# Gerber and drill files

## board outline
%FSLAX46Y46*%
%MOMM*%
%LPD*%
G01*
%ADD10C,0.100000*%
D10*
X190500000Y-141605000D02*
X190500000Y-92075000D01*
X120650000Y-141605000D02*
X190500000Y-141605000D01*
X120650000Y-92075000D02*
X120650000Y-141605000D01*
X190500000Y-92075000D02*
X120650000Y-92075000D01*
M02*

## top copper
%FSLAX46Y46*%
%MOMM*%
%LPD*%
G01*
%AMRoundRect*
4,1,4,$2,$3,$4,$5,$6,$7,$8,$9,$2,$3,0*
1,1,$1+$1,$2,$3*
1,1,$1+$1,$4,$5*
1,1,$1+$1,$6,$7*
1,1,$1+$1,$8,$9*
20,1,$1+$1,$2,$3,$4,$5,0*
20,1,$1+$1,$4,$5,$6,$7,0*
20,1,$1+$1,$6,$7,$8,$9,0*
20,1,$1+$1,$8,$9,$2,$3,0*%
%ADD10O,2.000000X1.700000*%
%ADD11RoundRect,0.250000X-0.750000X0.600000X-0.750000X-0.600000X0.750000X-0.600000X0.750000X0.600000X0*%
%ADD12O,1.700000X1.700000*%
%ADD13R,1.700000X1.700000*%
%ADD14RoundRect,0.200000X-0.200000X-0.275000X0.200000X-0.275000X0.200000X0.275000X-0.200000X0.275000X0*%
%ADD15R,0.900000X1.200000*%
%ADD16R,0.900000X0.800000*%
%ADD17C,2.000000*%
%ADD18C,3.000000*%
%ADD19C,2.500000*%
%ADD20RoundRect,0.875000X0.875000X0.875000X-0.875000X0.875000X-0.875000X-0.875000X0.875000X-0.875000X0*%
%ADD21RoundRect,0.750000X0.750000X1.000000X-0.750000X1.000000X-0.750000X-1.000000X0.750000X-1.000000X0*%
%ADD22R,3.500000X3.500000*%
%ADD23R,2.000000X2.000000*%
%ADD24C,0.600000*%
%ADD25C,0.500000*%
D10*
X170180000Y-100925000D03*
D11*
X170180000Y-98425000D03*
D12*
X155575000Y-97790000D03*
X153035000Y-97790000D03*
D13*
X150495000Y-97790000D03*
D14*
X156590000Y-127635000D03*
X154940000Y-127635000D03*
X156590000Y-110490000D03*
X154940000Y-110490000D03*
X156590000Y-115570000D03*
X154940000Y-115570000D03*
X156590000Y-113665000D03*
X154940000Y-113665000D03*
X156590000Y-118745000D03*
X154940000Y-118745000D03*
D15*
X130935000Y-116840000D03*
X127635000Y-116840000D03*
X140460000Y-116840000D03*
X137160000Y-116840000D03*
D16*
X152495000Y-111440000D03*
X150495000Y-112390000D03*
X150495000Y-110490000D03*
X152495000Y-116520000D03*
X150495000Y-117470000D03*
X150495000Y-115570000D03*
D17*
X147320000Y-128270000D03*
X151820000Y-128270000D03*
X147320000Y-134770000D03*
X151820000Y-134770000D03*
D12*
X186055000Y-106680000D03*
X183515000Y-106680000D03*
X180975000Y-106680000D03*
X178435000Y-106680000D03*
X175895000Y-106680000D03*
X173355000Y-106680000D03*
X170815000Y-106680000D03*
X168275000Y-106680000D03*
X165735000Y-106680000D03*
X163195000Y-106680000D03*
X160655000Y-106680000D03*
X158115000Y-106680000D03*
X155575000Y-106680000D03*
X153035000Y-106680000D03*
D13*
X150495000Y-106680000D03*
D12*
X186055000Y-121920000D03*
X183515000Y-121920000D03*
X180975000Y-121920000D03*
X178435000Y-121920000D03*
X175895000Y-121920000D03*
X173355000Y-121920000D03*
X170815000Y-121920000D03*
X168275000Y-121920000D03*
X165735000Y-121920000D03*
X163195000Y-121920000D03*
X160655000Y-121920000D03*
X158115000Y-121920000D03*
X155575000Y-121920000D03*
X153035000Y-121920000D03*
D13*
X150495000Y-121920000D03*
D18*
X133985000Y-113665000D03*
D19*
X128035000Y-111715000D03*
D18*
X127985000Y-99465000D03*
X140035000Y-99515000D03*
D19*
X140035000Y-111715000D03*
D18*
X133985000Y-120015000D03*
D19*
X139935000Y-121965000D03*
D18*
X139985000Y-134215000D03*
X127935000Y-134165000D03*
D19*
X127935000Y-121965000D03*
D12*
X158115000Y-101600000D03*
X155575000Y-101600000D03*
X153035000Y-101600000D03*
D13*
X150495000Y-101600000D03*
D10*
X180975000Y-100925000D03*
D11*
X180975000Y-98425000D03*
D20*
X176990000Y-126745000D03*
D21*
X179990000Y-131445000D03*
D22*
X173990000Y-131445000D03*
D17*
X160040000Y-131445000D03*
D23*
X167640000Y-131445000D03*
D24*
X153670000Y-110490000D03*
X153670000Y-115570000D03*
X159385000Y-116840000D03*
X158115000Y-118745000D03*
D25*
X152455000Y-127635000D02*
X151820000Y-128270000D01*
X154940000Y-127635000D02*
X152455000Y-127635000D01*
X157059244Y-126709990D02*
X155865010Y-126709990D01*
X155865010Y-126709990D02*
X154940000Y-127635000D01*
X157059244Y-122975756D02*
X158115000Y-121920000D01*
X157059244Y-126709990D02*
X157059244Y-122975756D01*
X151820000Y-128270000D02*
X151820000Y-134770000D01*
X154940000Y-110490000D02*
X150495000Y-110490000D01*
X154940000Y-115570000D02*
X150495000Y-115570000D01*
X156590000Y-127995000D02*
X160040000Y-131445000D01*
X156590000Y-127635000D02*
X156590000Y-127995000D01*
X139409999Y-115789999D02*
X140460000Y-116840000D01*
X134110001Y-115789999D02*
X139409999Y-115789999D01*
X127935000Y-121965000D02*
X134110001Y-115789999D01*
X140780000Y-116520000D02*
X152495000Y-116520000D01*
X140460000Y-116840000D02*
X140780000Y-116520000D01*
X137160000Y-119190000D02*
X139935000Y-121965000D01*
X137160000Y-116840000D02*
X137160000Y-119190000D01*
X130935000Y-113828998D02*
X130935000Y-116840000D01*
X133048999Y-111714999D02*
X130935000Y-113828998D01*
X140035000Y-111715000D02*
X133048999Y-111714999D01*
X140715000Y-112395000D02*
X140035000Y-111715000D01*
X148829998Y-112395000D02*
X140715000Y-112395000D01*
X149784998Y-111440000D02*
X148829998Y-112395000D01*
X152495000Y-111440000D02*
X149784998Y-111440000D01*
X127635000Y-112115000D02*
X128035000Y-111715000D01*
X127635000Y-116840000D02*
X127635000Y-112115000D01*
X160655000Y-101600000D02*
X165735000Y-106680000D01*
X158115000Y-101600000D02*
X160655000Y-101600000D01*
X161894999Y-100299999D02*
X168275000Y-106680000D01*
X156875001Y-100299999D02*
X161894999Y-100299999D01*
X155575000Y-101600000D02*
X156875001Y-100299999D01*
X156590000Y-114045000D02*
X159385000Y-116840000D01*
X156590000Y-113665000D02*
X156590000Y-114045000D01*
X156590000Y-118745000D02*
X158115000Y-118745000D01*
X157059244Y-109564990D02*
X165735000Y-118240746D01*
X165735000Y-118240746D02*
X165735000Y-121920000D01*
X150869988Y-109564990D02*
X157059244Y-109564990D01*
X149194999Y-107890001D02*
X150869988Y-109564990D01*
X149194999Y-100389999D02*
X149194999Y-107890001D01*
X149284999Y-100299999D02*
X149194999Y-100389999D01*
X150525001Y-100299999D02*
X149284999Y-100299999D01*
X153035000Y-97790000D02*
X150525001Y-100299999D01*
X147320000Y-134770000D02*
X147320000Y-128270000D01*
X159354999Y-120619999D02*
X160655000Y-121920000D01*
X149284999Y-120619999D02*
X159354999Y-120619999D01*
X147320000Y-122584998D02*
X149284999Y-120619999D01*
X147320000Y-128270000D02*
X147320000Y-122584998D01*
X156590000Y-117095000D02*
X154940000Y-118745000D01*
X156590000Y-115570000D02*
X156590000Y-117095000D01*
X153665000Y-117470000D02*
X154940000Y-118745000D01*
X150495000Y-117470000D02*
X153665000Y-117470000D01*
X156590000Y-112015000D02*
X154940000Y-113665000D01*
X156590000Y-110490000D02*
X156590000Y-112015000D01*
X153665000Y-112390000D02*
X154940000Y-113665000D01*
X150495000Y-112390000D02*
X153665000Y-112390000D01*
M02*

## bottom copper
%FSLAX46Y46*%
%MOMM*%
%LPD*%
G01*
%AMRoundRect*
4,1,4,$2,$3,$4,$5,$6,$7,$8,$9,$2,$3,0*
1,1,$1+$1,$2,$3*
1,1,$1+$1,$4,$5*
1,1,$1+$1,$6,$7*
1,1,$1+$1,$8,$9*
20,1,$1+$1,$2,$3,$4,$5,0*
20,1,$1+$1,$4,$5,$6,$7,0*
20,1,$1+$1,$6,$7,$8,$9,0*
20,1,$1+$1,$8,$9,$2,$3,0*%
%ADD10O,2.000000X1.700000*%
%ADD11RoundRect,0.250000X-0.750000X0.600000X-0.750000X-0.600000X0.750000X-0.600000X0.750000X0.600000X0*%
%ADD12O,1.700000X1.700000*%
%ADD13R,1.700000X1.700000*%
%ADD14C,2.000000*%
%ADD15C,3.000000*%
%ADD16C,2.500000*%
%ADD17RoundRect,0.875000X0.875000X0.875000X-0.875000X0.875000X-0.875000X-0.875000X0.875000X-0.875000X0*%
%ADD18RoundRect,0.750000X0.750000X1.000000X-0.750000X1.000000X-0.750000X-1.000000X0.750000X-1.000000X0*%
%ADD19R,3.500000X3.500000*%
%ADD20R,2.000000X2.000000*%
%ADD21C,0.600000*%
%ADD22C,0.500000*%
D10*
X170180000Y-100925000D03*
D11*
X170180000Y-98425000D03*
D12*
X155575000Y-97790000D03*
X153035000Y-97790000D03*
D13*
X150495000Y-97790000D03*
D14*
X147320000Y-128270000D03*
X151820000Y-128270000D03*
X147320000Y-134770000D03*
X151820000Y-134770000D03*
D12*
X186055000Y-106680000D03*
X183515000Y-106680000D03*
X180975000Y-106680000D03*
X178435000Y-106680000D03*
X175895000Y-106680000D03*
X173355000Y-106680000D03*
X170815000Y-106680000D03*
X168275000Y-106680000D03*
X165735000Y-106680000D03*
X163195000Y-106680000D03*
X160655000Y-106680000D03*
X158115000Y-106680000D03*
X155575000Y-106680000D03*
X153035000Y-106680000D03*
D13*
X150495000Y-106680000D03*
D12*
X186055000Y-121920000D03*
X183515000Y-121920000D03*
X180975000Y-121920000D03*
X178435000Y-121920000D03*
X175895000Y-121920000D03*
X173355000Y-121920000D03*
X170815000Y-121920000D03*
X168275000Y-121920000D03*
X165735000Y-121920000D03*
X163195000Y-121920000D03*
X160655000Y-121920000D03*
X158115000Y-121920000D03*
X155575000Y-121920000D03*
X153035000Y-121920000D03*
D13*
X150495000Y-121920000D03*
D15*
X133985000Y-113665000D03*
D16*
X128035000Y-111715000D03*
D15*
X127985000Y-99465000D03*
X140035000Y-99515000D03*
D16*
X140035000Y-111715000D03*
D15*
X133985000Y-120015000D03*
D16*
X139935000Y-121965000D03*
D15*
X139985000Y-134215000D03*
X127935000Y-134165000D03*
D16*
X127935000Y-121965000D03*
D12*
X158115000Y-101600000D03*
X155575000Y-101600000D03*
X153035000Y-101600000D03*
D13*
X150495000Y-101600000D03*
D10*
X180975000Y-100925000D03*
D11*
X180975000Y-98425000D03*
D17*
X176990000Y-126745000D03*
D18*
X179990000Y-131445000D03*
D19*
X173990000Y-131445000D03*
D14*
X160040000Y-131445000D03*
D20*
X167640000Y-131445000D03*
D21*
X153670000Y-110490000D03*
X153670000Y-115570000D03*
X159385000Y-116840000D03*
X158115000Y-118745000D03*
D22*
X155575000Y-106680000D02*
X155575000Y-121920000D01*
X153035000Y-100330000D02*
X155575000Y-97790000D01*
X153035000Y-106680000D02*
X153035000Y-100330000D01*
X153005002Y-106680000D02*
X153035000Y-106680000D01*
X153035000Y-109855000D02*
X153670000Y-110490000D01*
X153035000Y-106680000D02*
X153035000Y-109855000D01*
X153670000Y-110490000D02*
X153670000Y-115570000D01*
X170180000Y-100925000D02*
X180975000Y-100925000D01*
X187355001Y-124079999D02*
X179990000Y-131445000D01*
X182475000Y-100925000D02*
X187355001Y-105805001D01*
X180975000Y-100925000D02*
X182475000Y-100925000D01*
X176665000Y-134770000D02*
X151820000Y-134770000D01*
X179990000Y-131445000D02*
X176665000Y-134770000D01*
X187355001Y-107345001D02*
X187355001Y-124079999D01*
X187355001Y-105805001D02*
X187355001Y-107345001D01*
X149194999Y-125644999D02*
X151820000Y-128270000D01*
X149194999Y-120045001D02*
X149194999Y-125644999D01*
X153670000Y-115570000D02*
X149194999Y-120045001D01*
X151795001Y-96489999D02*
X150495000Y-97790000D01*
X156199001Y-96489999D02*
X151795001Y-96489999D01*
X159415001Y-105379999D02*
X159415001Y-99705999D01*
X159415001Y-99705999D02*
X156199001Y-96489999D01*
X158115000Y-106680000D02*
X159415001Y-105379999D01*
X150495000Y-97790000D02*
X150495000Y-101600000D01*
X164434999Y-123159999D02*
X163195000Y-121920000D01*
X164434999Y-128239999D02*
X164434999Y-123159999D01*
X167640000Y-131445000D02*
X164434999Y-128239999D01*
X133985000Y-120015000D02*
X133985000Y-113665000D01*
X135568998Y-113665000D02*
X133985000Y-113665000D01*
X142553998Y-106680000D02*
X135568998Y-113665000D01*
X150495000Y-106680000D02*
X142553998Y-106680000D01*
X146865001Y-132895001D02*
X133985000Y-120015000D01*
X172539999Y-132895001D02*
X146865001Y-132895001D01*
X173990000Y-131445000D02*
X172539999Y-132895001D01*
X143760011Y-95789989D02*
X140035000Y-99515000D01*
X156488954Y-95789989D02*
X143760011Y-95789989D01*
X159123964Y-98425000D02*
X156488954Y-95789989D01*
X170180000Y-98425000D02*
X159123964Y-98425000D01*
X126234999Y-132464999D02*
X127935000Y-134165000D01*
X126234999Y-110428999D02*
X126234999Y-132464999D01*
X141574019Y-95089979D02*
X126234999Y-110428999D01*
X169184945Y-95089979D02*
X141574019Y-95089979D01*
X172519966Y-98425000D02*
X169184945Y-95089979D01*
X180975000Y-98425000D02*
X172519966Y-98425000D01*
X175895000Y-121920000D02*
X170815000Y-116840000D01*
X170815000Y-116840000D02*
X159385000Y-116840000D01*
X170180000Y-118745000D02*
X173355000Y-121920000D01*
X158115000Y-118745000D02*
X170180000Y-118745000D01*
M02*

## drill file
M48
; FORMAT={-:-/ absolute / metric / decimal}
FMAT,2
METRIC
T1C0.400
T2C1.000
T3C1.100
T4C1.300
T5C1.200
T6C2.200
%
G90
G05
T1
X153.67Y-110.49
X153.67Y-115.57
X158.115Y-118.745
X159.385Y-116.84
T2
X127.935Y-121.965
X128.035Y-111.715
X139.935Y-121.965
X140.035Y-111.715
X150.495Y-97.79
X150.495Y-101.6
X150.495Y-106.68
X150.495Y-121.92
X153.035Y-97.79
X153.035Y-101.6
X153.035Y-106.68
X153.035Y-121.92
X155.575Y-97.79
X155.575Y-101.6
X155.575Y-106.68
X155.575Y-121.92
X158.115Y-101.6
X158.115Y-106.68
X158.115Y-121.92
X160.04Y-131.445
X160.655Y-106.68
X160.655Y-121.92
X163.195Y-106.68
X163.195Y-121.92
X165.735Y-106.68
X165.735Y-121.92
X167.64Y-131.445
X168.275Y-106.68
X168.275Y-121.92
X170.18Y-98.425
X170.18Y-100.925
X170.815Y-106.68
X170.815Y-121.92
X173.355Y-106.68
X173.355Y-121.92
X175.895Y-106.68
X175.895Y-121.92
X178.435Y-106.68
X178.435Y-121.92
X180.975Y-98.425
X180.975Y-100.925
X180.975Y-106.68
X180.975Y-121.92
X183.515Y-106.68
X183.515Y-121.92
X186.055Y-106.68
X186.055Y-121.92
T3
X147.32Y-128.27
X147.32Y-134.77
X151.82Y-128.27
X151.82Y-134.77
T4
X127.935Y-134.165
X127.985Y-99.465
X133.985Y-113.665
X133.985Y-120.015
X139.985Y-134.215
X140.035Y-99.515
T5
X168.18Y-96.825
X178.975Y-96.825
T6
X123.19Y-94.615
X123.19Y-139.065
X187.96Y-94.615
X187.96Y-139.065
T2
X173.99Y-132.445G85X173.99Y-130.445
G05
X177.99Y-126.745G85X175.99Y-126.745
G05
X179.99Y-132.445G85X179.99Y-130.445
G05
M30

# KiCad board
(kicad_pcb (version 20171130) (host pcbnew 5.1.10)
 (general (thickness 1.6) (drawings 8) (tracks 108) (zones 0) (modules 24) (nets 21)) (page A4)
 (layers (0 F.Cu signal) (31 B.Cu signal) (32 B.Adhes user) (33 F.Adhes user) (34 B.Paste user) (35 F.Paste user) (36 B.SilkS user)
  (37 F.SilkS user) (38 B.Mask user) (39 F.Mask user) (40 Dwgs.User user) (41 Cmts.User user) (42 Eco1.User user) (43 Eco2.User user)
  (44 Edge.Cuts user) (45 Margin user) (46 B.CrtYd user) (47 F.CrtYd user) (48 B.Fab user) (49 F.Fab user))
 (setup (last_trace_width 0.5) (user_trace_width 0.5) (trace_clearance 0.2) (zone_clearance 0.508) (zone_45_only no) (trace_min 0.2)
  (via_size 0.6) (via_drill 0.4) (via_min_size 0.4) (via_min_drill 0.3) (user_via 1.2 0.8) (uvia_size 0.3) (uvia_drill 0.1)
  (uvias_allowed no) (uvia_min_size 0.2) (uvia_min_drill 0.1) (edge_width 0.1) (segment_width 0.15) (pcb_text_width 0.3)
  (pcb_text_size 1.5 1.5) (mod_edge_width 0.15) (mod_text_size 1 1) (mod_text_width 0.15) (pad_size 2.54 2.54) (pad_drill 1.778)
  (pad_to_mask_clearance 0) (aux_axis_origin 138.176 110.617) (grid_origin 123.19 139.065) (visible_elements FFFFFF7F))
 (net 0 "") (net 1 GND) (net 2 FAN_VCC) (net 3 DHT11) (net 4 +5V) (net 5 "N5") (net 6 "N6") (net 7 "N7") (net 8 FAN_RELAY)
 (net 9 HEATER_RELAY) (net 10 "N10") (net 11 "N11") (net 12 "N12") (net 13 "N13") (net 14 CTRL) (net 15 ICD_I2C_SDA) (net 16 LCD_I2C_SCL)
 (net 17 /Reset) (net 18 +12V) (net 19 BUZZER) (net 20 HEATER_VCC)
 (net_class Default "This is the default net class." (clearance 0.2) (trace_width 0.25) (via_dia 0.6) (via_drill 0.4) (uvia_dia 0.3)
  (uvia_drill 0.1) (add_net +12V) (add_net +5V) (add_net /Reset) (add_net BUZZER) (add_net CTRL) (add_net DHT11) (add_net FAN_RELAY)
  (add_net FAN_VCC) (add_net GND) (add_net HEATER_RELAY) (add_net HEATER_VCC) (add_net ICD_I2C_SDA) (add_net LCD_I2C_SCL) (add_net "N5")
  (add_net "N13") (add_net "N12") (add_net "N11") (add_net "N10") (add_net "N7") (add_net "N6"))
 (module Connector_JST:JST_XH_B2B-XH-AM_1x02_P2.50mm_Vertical (layer F.Cu) (at 170.18 98.425 270)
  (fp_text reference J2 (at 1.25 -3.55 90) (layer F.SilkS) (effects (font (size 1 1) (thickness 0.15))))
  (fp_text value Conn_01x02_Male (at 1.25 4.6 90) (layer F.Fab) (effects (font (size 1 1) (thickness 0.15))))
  (pad "" np_thru_hole circle (at -1.6 2 270) (size 1.2 1.2) (drill 1.2) (layers *.Cu *.Mask))
  (pad 2 thru_hole oval (at 2.5 0 270) (size 1.7 2) (drill 1) (layers *.Cu *.Mask) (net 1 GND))
  (pad 1 thru_hole roundrect (at 0 0 270) (size 1.7 2) (drill 1) (layers *.Cu *.Mask) (roundrect_rratio 0.147059) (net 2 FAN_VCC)))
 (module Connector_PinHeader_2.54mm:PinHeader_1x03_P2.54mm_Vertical (layer F.Cu) (at 150.495 97.79 90)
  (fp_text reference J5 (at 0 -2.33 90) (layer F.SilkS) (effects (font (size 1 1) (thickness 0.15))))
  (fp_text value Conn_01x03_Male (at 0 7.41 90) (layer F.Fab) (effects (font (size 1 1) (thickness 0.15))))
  (pad 3 thru_hole oval (at 0 5.08 90) (size 1.7 1.7) (drill 1) (layers *.Cu *.Mask) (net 1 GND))
  (pad 2 thru_hole oval (at 0 2.54 90) (size 1.7 1.7) (drill 1) (layers *.Cu *.Mask) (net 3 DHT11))
  (pad 1 thru_hole rect (at 0 0 90) (size 1.7 1.7) (drill 1) (layers *.Cu *.Mask) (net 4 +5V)))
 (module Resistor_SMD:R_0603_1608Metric (layer F.Cu) (at 155.765 127.635)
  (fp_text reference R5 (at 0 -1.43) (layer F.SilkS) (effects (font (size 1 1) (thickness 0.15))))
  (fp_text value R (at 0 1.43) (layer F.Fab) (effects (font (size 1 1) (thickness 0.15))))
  (pad 2 smd roundrect (at 0.825 0) (size 0.8 0.95) (layers F.Cu F.Paste F.Mask) (roundrect_rratio 0.25) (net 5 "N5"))
  (pad 1 smd roundrect (at -0.825 0) (size 0.8 0.95) (layers F.Cu F.Paste F.Mask) (roundrect_rratio 0.25) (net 1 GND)))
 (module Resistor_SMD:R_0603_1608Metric (layer F.Cu) (at 155.765 110.49)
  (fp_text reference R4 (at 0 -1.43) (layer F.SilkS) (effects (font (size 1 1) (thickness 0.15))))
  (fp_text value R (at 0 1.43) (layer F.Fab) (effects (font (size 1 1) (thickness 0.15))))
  (pad 2 smd roundrect (at 0.825 0) (size 0.8 0.95) (layers F.Cu F.Paste F.Mask) (roundrect_rratio 0.25) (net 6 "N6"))
  (pad 1 smd roundrect (at -0.825 0) (size 0.8 0.95) (layers F.Cu F.Paste F.Mask) (roundrect_rratio 0.25) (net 1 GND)))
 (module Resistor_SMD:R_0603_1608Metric (layer F.Cu) (at 155.765 115.57)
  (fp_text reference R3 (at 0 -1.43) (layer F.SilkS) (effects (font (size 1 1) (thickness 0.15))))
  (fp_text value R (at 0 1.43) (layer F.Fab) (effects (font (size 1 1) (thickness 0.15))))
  (pad 2 smd roundrect (at 0.825 0) (size 0.8 0.95) (layers F.Cu F.Paste F.Mask) (roundrect_rratio 0.25) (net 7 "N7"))
  (pad 1 smd roundrect (at -0.825 0) (size 0.8 0.95) (layers F.Cu F.Paste F.Mask) (roundrect_rratio 0.25) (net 1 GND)))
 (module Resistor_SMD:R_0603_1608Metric (layer F.Cu) (at 155.765 113.665)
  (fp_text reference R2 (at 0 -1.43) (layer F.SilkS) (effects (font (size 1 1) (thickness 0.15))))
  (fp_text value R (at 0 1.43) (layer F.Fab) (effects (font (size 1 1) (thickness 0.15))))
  (pad 2 smd roundrect (at 0.825 0) (size 0.8 0.95) (layers F.Cu F.Paste F.Mask) (roundrect_rratio 0.25) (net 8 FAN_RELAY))
  (pad 1 smd roundrect (at -0.825 0) (size 0.8 0.95) (layers F.Cu F.Paste F.Mask) (roundrect_rratio 0.25) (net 6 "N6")))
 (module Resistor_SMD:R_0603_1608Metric (layer F.Cu) (at 155.765 118.745)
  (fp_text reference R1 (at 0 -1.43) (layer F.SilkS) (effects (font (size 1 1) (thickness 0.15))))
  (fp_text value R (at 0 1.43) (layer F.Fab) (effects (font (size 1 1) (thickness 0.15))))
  (pad 2 smd roundrect (at 0.825 0) (size 0.8 0.95) (layers F.Cu F.Paste F.Mask) (roundrect_rratio 0.25) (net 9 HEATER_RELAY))
  (pad 1 smd roundrect (at -0.825 0) (size 0.8 0.95) (layers F.Cu F.Paste F.Mask) (roundrect_rratio 0.25) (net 7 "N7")))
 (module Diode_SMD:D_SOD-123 (layer F.Cu) (at 129.285 116.84)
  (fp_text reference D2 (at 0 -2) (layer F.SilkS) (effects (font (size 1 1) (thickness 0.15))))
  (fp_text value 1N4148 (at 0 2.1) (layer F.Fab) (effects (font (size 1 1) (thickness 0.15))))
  (pad 2 smd rect (at 1.65 0) (size 0.9 1.2) (layers F.Cu F.Paste F.Mask) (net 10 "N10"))
  (pad 1 smd rect (at -1.65 0) (size 0.9 1.2) (layers F.Cu F.Paste F.Mask) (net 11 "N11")))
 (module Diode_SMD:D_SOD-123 (layer F.Cu) (at 138.81 116.84)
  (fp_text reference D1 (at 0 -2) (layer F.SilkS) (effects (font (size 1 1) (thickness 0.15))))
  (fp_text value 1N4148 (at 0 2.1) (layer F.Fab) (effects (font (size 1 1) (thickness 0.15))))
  (pad 2 smd rect (at 1.65 0) (size 0.9 1.2) (layers F.Cu F.Paste F.Mask) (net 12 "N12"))
  (pad 1 smd rect (at -1.65 0) (size 0.9 1.2) (layers F.Cu F.Paste F.Mask) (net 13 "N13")))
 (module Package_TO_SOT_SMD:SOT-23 (layer F.Cu) (at 151.495 111.44)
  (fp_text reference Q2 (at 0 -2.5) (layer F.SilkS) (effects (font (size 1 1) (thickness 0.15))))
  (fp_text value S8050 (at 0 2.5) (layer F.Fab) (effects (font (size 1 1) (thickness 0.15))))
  (pad 3 smd rect (at 1 0) (size 0.9 0.8) (layers F.Cu F.Paste F.Mask) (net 10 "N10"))
  (pad 2 smd rect (at -1 0.95) (size 0.9 0.8) (layers F.Cu F.Paste F.Mask) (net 6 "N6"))
  (pad 1 smd rect (at -1 -0.95) (size 0.9 0.8) (layers F.Cu F.Paste F.Mask) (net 1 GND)))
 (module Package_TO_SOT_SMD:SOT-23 (layer F.Cu) (at 151.495 116.52)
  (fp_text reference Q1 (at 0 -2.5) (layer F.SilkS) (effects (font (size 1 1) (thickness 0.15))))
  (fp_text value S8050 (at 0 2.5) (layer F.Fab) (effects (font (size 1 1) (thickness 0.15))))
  (pad 3 smd rect (at 1 0) (size 0.9 0.8) (layers F.Cu F.Paste F.Mask) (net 12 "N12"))
  (pad 2 smd rect (at -1 0.95) (size 0.9 0.8) (layers F.Cu F.Paste F.Mask) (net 7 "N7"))
  (pad 1 smd rect (at -1 -0.95) (size 0.9 0.8) (layers F.Cu F.Paste F.Mask) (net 1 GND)))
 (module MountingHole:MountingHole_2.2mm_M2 (layer F.Cu) (at 187.96 94.615)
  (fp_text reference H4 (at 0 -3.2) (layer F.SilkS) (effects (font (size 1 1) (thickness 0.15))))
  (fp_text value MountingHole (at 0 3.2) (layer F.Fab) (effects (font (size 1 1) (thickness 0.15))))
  (pad 1 np_thru_hole circle (at 0 0) (size 2.2 2.2) (drill 2.2) (layers *.Cu *.Mask)))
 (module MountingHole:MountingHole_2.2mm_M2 (layer F.Cu) (at 187.96 139.065)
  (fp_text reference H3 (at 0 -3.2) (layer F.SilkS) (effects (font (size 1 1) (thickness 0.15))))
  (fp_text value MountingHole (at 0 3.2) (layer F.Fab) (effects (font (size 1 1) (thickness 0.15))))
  (pad 1 np_thru_hole circle (at 0 0) (size 2.2 2.2) (drill 2.2) (layers *.Cu *.Mask)))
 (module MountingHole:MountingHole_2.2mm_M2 (layer F.Cu) (at 123.19 139.065)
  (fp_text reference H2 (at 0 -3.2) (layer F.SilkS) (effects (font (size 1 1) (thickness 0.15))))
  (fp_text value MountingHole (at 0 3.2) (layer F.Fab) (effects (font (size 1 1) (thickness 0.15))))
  (pad 1 np_thru_hole circle (at 0 0) (size 2.2 2.2) (drill 2.2) (layers *.Cu *.Mask)))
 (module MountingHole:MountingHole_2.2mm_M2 (layer F.Cu) (at 123.19 94.615)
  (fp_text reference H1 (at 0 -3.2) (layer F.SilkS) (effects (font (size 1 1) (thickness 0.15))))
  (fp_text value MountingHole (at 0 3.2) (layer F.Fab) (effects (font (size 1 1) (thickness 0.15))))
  (pad 1 np_thru_hole circle (at 0 0) (size 2.2 2.2) (drill 2.2) (layers *.Cu *.Mask)))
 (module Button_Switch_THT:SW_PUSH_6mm (layer F.Cu) (at 147.32 134.77 90)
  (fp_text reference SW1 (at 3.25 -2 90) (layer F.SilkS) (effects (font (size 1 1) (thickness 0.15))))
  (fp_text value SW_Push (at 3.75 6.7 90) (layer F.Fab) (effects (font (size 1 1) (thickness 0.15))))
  (pad 1 thru_hole circle (at 6.5 0 180) (size 2 2) (drill 1.1) (layers *.Cu *.Mask) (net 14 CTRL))
  (pad 2 thru_hole circle (at 6.5 4.5 180) (size 2 2) (drill 1.1) (layers *.Cu *.Mask) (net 1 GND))
  (pad 1 thru_hole circle (at 0 0 180) (size 2 2) (drill 1.1) (layers *.Cu *.Mask) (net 14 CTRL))
  (pad 2 thru_hole circle (at 0 4.5 180) (size 2 2) (drill 1.1) (layers *.Cu *.Mask) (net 1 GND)))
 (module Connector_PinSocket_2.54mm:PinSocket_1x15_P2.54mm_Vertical (layer F.Cu) (at 150.495 106.68 90)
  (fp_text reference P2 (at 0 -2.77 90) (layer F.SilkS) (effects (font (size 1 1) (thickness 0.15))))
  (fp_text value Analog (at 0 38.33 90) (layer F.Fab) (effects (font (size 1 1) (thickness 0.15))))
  (pad 15 thru_hole oval (at 0 35.56 90) (size 1.7 1.7) (drill 1) (layers *.Cu *.Mask))
  (pad 14 thru_hole oval (at 0 33.02 90) (size 1.7 1.7) (drill 1) (layers *.Cu *.Mask))
  (pad 13 thru_hole oval (at 0 30.48 90) (size 1.7 1.7) (drill 1) (layers *.Cu *.Mask))
  (pad 12 thru_hole oval (at 0 27.94 90) (size 1.7 1.7) (drill 1) (layers *.Cu *.Mask))
  (pad 11 thru_hole oval (at 0 25.4 90) (size 1.7 1.7) (drill 1) (layers *.Cu *.Mask))
  (pad 10 thru_hole oval (at 0 22.86 90) (size 1.7 1.7) (drill 1) (layers *.Cu *.Mask))
  (pad 9 thru_hole oval (at 0 20.32 90) (size 1.7 1.7) (drill 1) (layers *.Cu *.Mask))
  (pad 8 thru_hole oval (at 0 17.78 90) (size 1.7 1.7) (drill 1) (layers *.Cu *.Mask) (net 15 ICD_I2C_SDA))
  (pad 7 thru_hole oval (at 0 15.24 90) (size 1.7 1.7) (drill 1) (layers *.Cu *.Mask) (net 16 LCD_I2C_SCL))
  (pad 6 thru_hole oval (at 0 12.7 90) (size 1.7 1.7) (drill 1) (layers *.Cu *.Mask))
  (pad 5 thru_hole oval (at 0 10.16 90) (size 1.7 1.7) (drill 1) (layers *.Cu *.Mask))
  (pad 4 thru_hole oval (at 0 7.62 90) (size 1.7 1.7) (drill 1) (layers *.Cu *.Mask) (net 4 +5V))
  (pad 3 thru_hole oval (at 0 5.08 90) (size 1.7 1.7) (drill 1) (layers *.Cu *.Mask) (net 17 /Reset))
  (pad 2 thru_hole oval (at 0 2.54 90) (size 1.7 1.7) (drill 1) (layers *.Cu *.Mask) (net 1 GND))
  (pad 1 thru_hole rect (at 0 0 90) (size 1.7 1.7) (drill 1) (layers *.Cu *.Mask) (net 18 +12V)))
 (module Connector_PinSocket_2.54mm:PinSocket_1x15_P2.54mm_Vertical (layer F.Cu) (at 150.495 121.92 90)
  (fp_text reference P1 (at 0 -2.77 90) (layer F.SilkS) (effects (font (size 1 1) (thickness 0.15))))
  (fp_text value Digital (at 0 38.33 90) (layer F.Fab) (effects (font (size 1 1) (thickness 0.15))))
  (pad 15 thru_hole oval (at 0 35.56 90) (size 1.7 1.7) (drill 1) (layers *.Cu *.Mask))
  (pad 14 thru_hole oval (at 0 33.02 90) (size 1.7 1.7) (drill 1) (layers *.Cu *.Mask))
  (pad 13 thru_hole oval (at 0 30.48 90) (size 1.7 1.7) (drill 1) (layers *.Cu *.Mask))
  (pad 12 thru_hole oval (at 0 27.94 90) (size 1.7 1.7) (drill 1) (layers *.Cu *.Mask))
  (pad 11 thru_hole oval (at 0 25.4 90) (size 1.7 1.7) (drill 1) (layers *.Cu *.Mask) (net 8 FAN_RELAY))
  (pad 10 thru_hole oval (at 0 22.86 90) (size 1.7 1.7) (drill 1) (layers *.Cu *.Mask) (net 9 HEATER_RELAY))
  (pad 9 thru_hole oval (at 0 20.32 90) (size 1.7 1.7) (drill 1) (layers *.Cu *.Mask))
  (pad 8 thru_hole oval (at 0 17.78 90) (size 1.7 1.7) (drill 1) (layers *.Cu *.Mask))
  (pad 7 thru_hole oval (at 0 15.24 90) (size 1.7 1.7) (drill 1) (layers *.Cu *.Mask) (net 3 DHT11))
  (pad 6 thru_hole oval (at 0 12.7 90) (size 1.7 1.7) (drill 1) (layers *.Cu *.Mask) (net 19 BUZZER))
  (pad 5 thru_hole oval (at 0 10.16 90) (size 1.7 1.7) (drill 1) (layers *.Cu *.Mask) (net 14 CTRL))
  (pad 4 thru_hole oval (at 0 7.62 90) (size 1.7 1.7) (drill 1) (layers *.Cu *.Mask) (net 1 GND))
  (pad 3 thru_hole oval (at 0 5.08 90) (size 1.7 1.7) (drill 1) (layers *.Cu *.Mask) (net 17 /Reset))
  (pad 2 thru_hole oval (at 0 2.54 90) (size 1.7 1.7) (drill 1) (layers *.Cu *.Mask))
  (pad 1 thru_hole rect (at 0 0 90) (size 1.7 1.7) (drill 1) (layers *.Cu *.Mask)))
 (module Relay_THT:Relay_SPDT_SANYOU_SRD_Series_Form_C (layer F.Cu) (at 133.985 113.665 90)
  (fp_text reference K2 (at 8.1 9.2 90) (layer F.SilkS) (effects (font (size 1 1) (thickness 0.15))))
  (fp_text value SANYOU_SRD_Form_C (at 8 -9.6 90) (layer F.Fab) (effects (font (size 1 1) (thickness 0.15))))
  (pad 1 thru_hole circle (at 0 0 180) (size 3 3) (drill 1.3) (layers *.Cu *.Mask) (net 18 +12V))
  (pad 5 thru_hole circle (at 1.95 -5.95 180) (size 2.5 2.5) (drill 1) (layers *.Cu *.Mask) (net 11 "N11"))
  (pad 4 thru_hole circle (at 14.2 -6 180) (size 3 3) (drill 1.3) (layers *.Cu *.Mask))
  (pad 3 thru_hole circle (at 14.15 6.05 180) (size 3 3) (drill 1.3) (layers *.Cu *.Mask) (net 2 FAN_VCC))
  (pad 2 thru_hole circle (at 1.95 6.05 180) (size 2.5 2.5) (drill 1) (layers *.Cu *.Mask) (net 10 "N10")))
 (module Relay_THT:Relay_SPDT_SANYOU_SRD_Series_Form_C (layer F.Cu) (at 133.985 120.015 270)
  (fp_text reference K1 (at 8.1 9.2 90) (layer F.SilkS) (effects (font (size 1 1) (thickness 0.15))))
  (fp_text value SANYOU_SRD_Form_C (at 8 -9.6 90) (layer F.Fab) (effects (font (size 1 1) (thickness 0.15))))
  (pad 1 thru_hole circle (at 0 0) (size 3 3) (drill 1.3) (layers *.Cu *.Mask) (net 18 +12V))
  (pad 5 thru_hole circle (at 1.95 -5.95) (size 2.5 2.5) (drill 1) (layers *.Cu *.Mask) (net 13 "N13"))
  (pad 4 thru_hole circle (at 14.2 -6) (size 3 3) (drill 1.3) (layers *.Cu *.Mask))
  (pad 3 thru_hole circle (at 14.15 6.05) (size 3 3) (drill 1.3) (layers *.Cu *.Mask) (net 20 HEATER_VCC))
  (pad 2 thru_hole circle (at 1.95 6.05) (size 2.5 2.5) (drill 1) (layers *.Cu *.Mask) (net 12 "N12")))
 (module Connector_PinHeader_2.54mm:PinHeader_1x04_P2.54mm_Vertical (layer F.Cu) (at 150.495 101.6 90)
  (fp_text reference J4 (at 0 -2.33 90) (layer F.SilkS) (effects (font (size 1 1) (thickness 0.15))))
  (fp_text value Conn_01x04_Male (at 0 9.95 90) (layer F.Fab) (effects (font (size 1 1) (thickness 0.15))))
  (pad 4 thru_hole oval (at 0 7.62 90) (size 1.7 1.7) (drill 1) (layers *.Cu *.Mask) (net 16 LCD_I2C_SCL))
  (pad 3 thru_hole oval (at 0 5.08 90) (size 1.7 1.7) (drill 1) (layers *.Cu *.Mask) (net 15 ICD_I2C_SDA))
  (pad 2 thru_hole oval (at 0 2.54 90) (size 1.7 1.7) (drill 1) (layers *.Cu *.Mask) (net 1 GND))
  (pad 1 thru_hole rect (at 0 0 90) (size 1.7 1.7) (drill 1) (layers *.Cu *.Mask) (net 4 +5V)))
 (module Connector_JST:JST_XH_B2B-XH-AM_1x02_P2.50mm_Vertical (layer F.Cu) (at 180.975 98.425 270)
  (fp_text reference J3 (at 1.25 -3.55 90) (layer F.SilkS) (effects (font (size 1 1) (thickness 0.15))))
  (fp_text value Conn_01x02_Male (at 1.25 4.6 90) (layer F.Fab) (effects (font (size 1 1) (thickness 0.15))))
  (pad "" np_thru_hole circle (at -1.6 2 270) (size 1.2 1.2) (drill 1.2) (layers *.Cu *.Mask))
  (pad 2 thru_hole oval (at 2.5 0 270) (size 1.7 2) (drill 1) (layers *.Cu *.Mask) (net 1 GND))
  (pad 1 thru_hole roundrect (at 0 0 270) (size 1.7 2) (drill 1) (layers *.Cu *.Mask) (roundrect_rratio 0.147059) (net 20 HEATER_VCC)))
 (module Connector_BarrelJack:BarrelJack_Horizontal (layer F.Cu) (at 173.99 131.445 180)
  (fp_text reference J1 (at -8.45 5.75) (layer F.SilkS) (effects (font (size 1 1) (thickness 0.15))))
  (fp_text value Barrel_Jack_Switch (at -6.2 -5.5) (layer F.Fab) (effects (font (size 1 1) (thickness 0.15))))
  (pad 3 thru_hole roundrect (at -3 4.7 180) (size 3.5 3.5) (drill oval 3 1) (layers *.Cu *.Mask) (roundrect_rratio 0.25))
  (pad 2 thru_hole roundrect (at -6 0 180) (size 3 3.5) (drill oval 1 3) (layers *.Cu *.Mask) (roundrect_rratio 0.25) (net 1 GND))
  (pad 1 thru_hole rect (at 0 0 180) (size 3.5 3.5) (drill oval 1 3) (layers *.Cu *.Mask) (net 18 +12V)))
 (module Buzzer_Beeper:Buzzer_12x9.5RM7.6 (layer F.Cu) (at 167.64 131.445 180)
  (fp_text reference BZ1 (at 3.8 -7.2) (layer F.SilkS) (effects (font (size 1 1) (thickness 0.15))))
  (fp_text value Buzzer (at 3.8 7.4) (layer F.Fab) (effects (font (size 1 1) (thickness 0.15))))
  (pad 2 thru_hole circle (at 7.6 0 180) (size 2 2) (drill 1) (layers *.Cu *.Mask) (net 5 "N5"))
  (pad 1 thru_hole rect (at 0 0 180) (size 2 2) (drill 1) (layers *.Cu *.Mask) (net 19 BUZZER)))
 (gr_line (start 190.5 141.605) (end 190.5 92.075) (angle 90) (layer Edge.Cuts) (width 0.1))
 (gr_line (start 120.65 141.605) (end 190.5 141.605) (angle 90) (layer Edge.Cuts) (width 0.1))
 (gr_line (start 120.65 92.075) (end 120.65 141.605) (angle 90) (layer Edge.Cuts) (width 0.1))
 (gr_line (start 190.5 92.075) (end 120.65 92.075) (angle 90) (layer Edge.Cuts) (width 0.1))
 (segment (start 155.575 106.68) (end 155.575 121.92) (width 0.5) (layer B.Cu) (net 17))
 (via (at 153.67 110.49) (size 0.6) (drill 0.4) (layers F.Cu B.Cu) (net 1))
 (via (at 153.67 115.57) (size 0.6) (drill 0.4) (layers F.Cu B.Cu) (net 1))
 (via (at 159.385 116.84) (size 0.6) (drill 0.4) (layers F.Cu B.Cu) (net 8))
 (via (at 158.115 118.745) (size 0.6) (drill 0.4) (layers F.Cu B.Cu) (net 9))
 (segment (start 153.035 100.33) (end 155.575 97.79) (width 0.5) (layer B.Cu) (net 1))
 (segment (start 153.035 106.68) (end 153.035 100.33) (width 0.5) (layer B.Cu) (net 1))
 (segment (start 152.455 127.635) (end 151.82 128.27) (width 0.5) (layer F.Cu) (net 1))
 (segment (start 154.94 127.635) (end 152.455 127.635) (width 0.5) (layer F.Cu) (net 1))
 (segment (start 157.059244 126.70999) (end 155.86501 126.70999) (width 0.5) (layer F.Cu) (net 1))
 (segment (start 155.86501 126.70999) (end 154.94 127.635) (width 0.5) (layer F.Cu) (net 1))
 (segment (start 157.059244 122.975756) (end 158.115 121.92) (width 0.5) (layer F.Cu) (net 1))
 (segment (start 157.059244 126.70999) (end 157.059244 122.975756) (width 0.5) (layer F.Cu) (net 1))
 (segment (start 151.82 128.27) (end 151.82 134.77) (width 0.5) (layer F.Cu) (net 1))
 (segment (start 153.005002 106.68) (end 153.035 106.68) (width 0.5) (layer B.Cu) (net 1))
 (segment (start 154.94 110.49) (end 150.495 110.49) (width 0.5) (layer F.Cu) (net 1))
 (segment (start 154.94 115.57) (end 150.495 115.57) (width 0.5) (layer F.Cu) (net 1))
 (segment (start 153.035 109.855) (end 153.67 110.49) (width 0.5) (layer B.Cu) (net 1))
 (segment (start 153.035 106.68) (end 153.035 109.855) (width 0.5) (layer B.Cu) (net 1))
 (segment (start 153.67 110.49) (end 153.67 115.57) (width 0.5) (layer B.Cu) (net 1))
 (segment (start 170.18 100.925) (end 180.975 100.925) (width 0.5) (layer B.Cu) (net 1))
 (segment (start 187.355001 124.079999) (end 179.99 131.445) (width 0.5) (layer B.Cu) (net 1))
 (segment (start 182.475 100.925) (end 187.355001 105.805001) (width 0.5) (layer B.Cu) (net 1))
 (segment (start 180.975 100.925) (end 182.475 100.925) (width 0.5) (layer B.Cu) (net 1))
 (segment (start 176.665 134.77) (end 151.82 134.77) (width 0.5) (layer B.Cu) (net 1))
 (segment (start 179.99 131.445) (end 176.665 134.77) (width 0.5) (layer B.Cu) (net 1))
 (segment (start 187.355001 107.345001) (end 187.355001 124.079999) (width 0.5) (layer B.Cu) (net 1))
 (segment (start 187.355001 105.805001) (end 187.355001 107.345001) (width 0.5) (layer B.Cu) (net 1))
 (segment (start 149.194999 125.644999) (end 151.82 128.27) (width 0.5) (layer B.Cu) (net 1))
 (segment (start 149.194999 120.045001) (end 149.194999 125.644999) (width 0.5) (layer B.Cu) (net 1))
 (segment (start 153.67 115.57) (end 149.194999 120.045001) (width 0.5) (layer B.Cu) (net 1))
 (segment (start 151.795001 96.489999) (end 150.495 97.79) (width 0.5) (layer B.Cu) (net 4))
 (segment (start 156.199001 96.489999) (end 151.795001 96.489999) (width 0.5) (layer B.Cu) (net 4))
 (segment (start 159.415001 105.379999) (end 159.415001 99.705999) (width 0.5) (layer B.Cu) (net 4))
 (segment (start 159.415001 99.705999) (end 156.199001 96.489999) (width 0.5) (layer B.Cu) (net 4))
 (segment (start 158.115 106.68) (end 159.415001 105.379999) (width 0.5) (layer B.Cu) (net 4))
 (segment (start 150.495 97.79) (end 150.495 101.6) (width 0.5) (layer B.Cu) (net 4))
 (segment (start 156.59 127.995) (end 160.04 131.445) (width 0.5) (layer F.Cu) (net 5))
 (segment (start 156.59 127.635) (end 156.59 127.995) (width 0.5) (layer F.Cu) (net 5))
 (segment (start 164.434999 123.159999) (end 163.195 121.92) (width 0.5) (layer B.Cu) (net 19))
 (segment (start 164.434999 128.239999) (end 164.434999 123.159999) (width 0.5) (layer B.Cu) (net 19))
 (segment (start 167.64 131.445) (end 164.434999 128.239999) (width 0.5) (layer B.Cu) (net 19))
 (segment (start 139.409999 115.789999) (end 140.46 116.84) (width 0.5) (layer F.Cu) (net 12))
 (segment (start 134.110001 115.789999) (end 139.409999 115.789999) (width 0.5) (layer F.Cu) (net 12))
 (segment (start 127.935 121.965) (end 134.110001 115.789999) (width 0.5) (layer F.Cu) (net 12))
 (segment (start 140.78 116.52) (end 152.495 116.52) (width 0.5) (layer F.Cu) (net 12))
 (segment (start 140.46 116.84) (end 140.78 116.52) (width 0.5) (layer F.Cu) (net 12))
 (segment (start 137.16 119.19) (end 139.935 121.965) (width 0.5) (layer F.Cu) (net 13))
 (segment (start 137.16 116.84) (end 137.16 119.19) (width 0.5) (layer F.Cu) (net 13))
 (segment (start 130.935 113.828998) (end 130.935 116.84) (width 0.5) (layer F.Cu) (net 10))
 (segment (start 133.048999 111.714999) (end 130.935 113.828998) (width 0.5) (layer F.Cu) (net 10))
 (segment (start 140.035 111.715) (end 133.048999 111.714999) (width 0.5) (layer F.Cu) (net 10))
 (segment (start 140.715 112.395) (end 140.035 111.715) (width 0.5) (layer F.Cu) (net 10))
 (segment (start 148.829998 112.395) (end 140.715 112.395) (width 0.5) (layer F.Cu) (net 10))
 (segment (start 149.784998 111.44) (end 148.829998 112.395) (width 0.5) (layer F.Cu) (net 10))
 (segment (start 152.495 111.44) (end 149.784998 111.44) (width 0.5) (layer F.Cu) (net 10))
 (segment (start 127.635 112.115) (end 128.035 111.715) (width 0.5) (layer F.Cu) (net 11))
 (segment (start 127.635 116.84) (end 127.635 112.115) (width 0.5) (layer F.Cu) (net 11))
 (segment (start 133.985 120.015) (end 133.985 113.665) (width 0.5) (layer B.Cu) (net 18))
 (segment (start 135.568998 113.665) (end 133.985 113.665) (width 0.5) (layer B.Cu) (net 18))
 (segment (start 142.553998 106.68) (end 135.568998 113.665) (width 0.5) (layer B.Cu) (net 18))
 (segment (start 150.495 106.68) (end 142.553998 106.68) (width 0.5) (layer B.Cu) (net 18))
 (segment (start 146.865001 132.895001) (end 133.985 120.015) (width 0.5) (layer B.Cu) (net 18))
 (segment (start 172.539999 132.895001) (end 146.865001 132.895001) (width 0.5) (layer B.Cu) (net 18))
 (segment (start 173.99 131.445) (end 172.539999 132.895001) (width 0.5) (layer B.Cu) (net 18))
 (segment (start 143.760011 95.789989) (end 140.035 99.515) (width 0.5) (layer B.Cu) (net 2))
 (segment (start 156.488954 95.789989) (end 143.760011 95.789989) (width 0.5) (layer B.Cu) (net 2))
 (segment (start 159.123964 98.425) (end 156.488954 95.789989) (width 0.5) (layer B.Cu) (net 2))
 (segment (start 170.18 98.425) (end 159.123964 98.425) (width 0.5) (layer B.Cu) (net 2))
 (segment (start 126.234999 132.464999) (end 127.935 134.165) (width 0.5) (layer B.Cu) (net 20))
 (segment (start 126.234999 110.428999) (end 126.234999 132.464999) (width 0.5) (layer B.Cu) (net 20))
 (segment (start 141.574019 95.089979) (end 126.234999 110.428999) (width 0.5) (layer B.Cu) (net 20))
 (segment (start 169.184945 95.089979) (end 141.574019 95.089979) (width 0.5) (layer B.Cu) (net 20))
 (segment (start 172.519966 98.425) (end 169.184945 95.089979) (width 0.5) (layer B.Cu) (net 20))
 (segment (start 180.975 98.425) (end 172.519966 98.425) (width 0.5) (layer B.Cu) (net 20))
 (segment (start 160.655 101.6) (end 165.735 106.68) (width 0.5) (layer F.Cu) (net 16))
 (segment (start 158.115 101.6) (end 160.655 101.6) (width 0.5) (layer F.Cu) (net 16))
 (segment (start 161.894999 100.299999) (end 168.275 106.68) (width 0.5) (layer F.Cu) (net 15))
 (segment (start 156.875001 100.299999) (end 161.894999 100.299999) (width 0.5) (layer F.Cu) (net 15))
 (segment (start 155.575 101.6) (end 156.875001 100.299999) (width 0.5) (layer F.Cu) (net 15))
 (segment (start 175.895 121.92) (end 170.815 116.84) (width 0.5) (layer B.Cu) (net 8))
 (segment (start 170.815 116.84) (end 159.385 116.84) (width 0.5) (layer B.Cu) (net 8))
 (segment (start 156.59 114.045) (end 159.385 116.84) (width 0.5) (layer F.Cu) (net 8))
 (segment (start 156.59 113.665) (end 156.59 114.045) (width 0.5) (layer F.Cu) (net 8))
 (segment (start 156.59 118.745) (end 158.115 118.745) (width 0.5) (layer F.Cu) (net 9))
 (segment (start 170.18 118.745) (end 173.355 121.92) (width 0.5) (layer B.Cu) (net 9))
 (segment (start 158.115 118.745) (end 170.18 118.745) (width 0.5) (layer B.Cu) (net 9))
 (segment (start 157.059244 109.56499) (end 165.735 118.240746) (width 0.5) (layer F.Cu) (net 3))
 (segment (start 165.735 118.240746) (end 165.735 121.92) (width 0.5) (layer F.Cu) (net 3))
 (segment (start 150.869988 109.56499) (end 157.059244 109.56499) (width 0.5) (layer F.Cu) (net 3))
 (segment (start 149.194999 107.890001) (end 150.869988 109.56499) (width 0.5) (layer F.Cu) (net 3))
 (segment (start 149.194999 100.389999) (end 149.194999 107.890001) (width 0.5) (layer F.Cu) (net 3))
 (segment (start 149.284999 100.299999) (end 149.194999 100.389999) (width 0.5) (layer F.Cu) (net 3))
 (segment (start 150.525001 100.299999) (end 149.284999 100.299999) (width 0.5) (layer F.Cu) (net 3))
 (segment (start 153.035 97.79) (end 150.525001 100.299999) (width 0.5) (layer F.Cu) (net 3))
 (segment (start 147.32 134.77) (end 147.32 128.27) (width 0.5) (layer F.Cu) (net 14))
 (segment (start 159.354999 120.619999) (end 160.655 121.92) (width 0.5) (layer F.Cu) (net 14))
 (segment (start 149.284999 120.619999) (end 159.354999 120.619999) (width 0.5) (layer F.Cu) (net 14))
 (segment (start 147.32 122.584998) (end 149.284999 120.619999) (width 0.5) (layer F.Cu) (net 14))
 (segment (start 147.32 128.27) (end 147.32 122.584998) (width 0.5) (layer F.Cu) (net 14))
 (segment (start 156.59 117.095) (end 154.94 118.745) (width 0.5) (layer F.Cu) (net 7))
 (segment (start 156.59 115.57) (end 156.59 117.095) (width 0.5) (layer F.Cu) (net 7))
 (segment (start 153.665 117.47) (end 154.94 118.745) (width 0.5) (layer F.Cu) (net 7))
 (segment (start 150.495 117.47) (end 153.665 117.47) (width 0.5) (layer F.Cu) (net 7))
 (segment (start 156.59 112.015) (end 154.94 113.665) (width 0.5) (layer F.Cu) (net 6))
 (segment (start 156.59 110.49) (end 156.59 112.015) (width 0.5) (layer F.Cu) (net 6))
 (segment (start 153.665 112.39) (end 154.94 113.665) (width 0.5) (layer F.Cu) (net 6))
 (segment (start 150.495 112.39) (end 153.665 112.39) (width 0.5) (layer F.Cu) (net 6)))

